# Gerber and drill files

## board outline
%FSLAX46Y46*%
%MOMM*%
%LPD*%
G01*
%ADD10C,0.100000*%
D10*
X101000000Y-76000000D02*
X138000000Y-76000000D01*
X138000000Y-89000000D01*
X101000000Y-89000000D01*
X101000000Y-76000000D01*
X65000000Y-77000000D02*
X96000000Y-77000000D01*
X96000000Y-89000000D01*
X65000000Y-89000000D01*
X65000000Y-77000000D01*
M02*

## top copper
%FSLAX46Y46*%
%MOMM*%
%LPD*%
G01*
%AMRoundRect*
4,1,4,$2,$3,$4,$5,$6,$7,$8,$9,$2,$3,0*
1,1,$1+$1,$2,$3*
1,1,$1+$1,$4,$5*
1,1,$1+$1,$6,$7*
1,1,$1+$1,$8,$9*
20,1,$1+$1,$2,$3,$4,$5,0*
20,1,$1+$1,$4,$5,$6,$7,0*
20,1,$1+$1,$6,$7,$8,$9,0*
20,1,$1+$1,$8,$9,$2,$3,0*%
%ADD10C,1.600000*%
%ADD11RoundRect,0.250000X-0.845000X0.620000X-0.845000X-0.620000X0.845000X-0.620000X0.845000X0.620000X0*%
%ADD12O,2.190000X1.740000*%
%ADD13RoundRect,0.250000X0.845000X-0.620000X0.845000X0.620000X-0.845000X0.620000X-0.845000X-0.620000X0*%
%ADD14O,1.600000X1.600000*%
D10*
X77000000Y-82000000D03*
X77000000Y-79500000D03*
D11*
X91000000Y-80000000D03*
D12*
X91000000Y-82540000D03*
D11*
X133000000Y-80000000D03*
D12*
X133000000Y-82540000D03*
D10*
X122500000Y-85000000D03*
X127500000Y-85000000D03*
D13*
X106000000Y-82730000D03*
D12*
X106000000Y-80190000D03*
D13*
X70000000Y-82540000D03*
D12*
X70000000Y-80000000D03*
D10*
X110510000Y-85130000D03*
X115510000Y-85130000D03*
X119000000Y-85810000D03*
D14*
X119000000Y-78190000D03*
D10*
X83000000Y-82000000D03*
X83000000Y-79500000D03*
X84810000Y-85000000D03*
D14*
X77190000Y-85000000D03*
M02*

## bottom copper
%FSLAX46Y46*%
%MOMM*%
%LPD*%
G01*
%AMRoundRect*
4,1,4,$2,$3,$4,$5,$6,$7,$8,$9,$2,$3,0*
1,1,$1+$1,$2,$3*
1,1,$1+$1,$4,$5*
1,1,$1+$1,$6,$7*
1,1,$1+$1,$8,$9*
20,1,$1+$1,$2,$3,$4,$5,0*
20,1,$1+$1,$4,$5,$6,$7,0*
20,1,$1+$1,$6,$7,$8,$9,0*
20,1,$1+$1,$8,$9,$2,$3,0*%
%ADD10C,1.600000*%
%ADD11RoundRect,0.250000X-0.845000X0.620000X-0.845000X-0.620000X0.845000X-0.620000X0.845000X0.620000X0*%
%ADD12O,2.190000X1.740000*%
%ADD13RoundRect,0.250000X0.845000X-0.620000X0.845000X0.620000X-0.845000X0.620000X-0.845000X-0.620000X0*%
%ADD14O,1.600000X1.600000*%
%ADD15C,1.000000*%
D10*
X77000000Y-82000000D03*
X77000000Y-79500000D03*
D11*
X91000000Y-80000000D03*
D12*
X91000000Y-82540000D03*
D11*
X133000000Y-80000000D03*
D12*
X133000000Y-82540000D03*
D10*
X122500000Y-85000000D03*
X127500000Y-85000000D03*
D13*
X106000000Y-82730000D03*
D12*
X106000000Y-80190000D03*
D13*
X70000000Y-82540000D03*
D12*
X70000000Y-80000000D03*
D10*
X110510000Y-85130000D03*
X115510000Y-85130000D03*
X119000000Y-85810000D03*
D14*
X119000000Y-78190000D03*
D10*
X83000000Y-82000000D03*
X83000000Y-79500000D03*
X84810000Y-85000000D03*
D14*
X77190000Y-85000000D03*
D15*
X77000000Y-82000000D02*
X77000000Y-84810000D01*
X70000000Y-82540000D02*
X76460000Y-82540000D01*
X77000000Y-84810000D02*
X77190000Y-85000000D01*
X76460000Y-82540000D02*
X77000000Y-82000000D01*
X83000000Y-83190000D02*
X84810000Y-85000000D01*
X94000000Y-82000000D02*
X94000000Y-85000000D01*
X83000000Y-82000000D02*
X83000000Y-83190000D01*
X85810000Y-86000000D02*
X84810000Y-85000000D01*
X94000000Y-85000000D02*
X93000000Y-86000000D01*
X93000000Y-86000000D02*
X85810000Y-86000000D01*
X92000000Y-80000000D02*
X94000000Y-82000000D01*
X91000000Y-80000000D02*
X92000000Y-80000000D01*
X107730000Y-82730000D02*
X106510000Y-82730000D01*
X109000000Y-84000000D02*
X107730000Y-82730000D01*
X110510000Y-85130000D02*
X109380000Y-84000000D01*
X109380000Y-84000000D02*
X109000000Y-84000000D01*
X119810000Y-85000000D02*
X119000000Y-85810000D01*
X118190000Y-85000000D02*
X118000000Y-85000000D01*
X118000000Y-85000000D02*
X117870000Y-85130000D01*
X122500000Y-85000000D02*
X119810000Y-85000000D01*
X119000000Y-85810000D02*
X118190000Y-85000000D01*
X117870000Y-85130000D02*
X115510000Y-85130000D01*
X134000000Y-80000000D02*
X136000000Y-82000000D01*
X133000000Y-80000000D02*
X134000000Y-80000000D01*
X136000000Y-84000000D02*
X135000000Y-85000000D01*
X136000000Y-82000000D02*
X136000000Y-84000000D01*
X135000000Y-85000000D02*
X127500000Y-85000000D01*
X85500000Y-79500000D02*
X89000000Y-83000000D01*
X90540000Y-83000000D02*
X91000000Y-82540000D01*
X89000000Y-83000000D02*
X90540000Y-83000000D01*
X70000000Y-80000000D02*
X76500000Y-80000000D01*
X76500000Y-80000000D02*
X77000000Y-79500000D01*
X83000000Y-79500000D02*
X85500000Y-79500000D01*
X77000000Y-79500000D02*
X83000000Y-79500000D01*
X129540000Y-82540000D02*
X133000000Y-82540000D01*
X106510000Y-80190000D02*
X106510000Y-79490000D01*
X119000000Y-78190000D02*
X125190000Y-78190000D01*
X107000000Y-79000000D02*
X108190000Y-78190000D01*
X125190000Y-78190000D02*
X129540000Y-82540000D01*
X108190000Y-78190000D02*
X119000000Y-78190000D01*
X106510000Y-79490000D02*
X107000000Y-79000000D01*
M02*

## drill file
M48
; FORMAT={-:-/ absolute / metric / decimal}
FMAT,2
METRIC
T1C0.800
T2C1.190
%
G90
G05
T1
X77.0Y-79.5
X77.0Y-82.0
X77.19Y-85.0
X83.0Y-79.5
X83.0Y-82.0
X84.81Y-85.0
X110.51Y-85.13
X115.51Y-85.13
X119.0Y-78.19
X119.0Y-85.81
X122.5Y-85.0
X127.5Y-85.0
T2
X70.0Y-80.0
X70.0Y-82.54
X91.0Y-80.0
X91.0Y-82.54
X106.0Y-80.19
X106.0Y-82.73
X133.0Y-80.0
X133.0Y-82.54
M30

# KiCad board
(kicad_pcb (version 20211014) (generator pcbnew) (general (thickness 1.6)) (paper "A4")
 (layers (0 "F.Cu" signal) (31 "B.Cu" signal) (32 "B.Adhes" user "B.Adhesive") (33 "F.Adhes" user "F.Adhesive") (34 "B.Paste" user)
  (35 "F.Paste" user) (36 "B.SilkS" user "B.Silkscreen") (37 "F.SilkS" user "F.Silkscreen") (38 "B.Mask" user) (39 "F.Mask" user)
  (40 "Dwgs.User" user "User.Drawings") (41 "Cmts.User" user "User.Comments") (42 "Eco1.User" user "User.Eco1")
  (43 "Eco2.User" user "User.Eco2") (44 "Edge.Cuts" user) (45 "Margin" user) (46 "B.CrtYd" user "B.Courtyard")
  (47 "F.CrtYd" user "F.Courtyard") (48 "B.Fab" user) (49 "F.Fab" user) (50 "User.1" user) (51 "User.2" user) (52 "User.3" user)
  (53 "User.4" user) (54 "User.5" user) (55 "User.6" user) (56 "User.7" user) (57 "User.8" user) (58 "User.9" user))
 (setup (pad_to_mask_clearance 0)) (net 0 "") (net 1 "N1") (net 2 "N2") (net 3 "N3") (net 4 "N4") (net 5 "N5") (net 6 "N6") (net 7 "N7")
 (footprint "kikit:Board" (layer "F.Cu") (at 67 77)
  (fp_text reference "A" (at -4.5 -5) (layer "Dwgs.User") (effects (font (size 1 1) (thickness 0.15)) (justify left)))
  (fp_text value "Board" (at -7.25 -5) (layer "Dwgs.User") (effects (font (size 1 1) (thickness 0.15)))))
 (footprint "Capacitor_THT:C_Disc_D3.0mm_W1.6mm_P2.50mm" (layer "F.Cu") (at 77 82 90)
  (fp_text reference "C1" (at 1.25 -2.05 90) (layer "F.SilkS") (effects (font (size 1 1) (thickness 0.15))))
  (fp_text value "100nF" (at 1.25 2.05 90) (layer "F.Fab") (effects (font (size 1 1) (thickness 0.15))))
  (pad "1" thru_hole circle (at 0 0 90) (size 1.6 1.6) (drill 0.8) (layers *.Cu *.Mask) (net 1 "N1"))
  (pad "2" thru_hole circle (at 2.5 0 90) (size 1.6 1.6) (drill 0.8) (layers *.Cu *.Mask) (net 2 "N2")))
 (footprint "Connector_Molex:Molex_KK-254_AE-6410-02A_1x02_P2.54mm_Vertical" (layer "F.Cu") (at 91 80 -90)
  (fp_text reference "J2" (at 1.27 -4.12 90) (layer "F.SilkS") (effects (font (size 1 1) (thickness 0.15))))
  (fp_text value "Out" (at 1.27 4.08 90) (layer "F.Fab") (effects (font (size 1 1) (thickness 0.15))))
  (pad "1" thru_hole roundrect (at 0 0 270) (size 1.74 2.19) (drill 1.19) (layers *.Cu *.Mask) (roundrect_rratio 0.143678) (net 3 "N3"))
  (pad "2" thru_hole oval (at 2.54 0 270) (size 1.74 2.19) (drill 1.19) (layers *.Cu *.Mask) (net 2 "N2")))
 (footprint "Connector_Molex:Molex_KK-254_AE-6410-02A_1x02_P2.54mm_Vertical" (layer "F.Cu") (at 133 80 -90)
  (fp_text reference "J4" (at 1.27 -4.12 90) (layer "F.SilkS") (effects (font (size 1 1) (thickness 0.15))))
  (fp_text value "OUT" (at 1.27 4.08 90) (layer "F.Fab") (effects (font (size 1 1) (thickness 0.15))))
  (pad "1" thru_hole roundrect (at 0 0 270) (size 1.74 2.19) (drill 1.19) (layers *.Cu *.Mask) (roundrect_rratio 0.143678) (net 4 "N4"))
  (pad "2" thru_hole oval (at 2.54 0 270) (size 1.74 2.19) (drill 1.19) (layers *.Cu *.Mask) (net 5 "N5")))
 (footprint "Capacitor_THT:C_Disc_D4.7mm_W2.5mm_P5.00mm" (layer "F.Cu") (at 122.5 85)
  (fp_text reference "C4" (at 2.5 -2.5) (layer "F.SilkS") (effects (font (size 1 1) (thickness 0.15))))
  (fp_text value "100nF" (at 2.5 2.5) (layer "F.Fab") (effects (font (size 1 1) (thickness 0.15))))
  (pad "1" thru_hole circle (at 0 0) (size 1.6 1.6) (drill 0.8) (layers *.Cu *.Mask) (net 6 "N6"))
  (pad "2" thru_hole circle (at 5 0) (size 1.6 1.6) (drill 0.8) (layers *.Cu *.Mask) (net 4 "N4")))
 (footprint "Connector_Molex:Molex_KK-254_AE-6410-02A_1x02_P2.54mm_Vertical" (layer "F.Cu") (at 106 82.73 90)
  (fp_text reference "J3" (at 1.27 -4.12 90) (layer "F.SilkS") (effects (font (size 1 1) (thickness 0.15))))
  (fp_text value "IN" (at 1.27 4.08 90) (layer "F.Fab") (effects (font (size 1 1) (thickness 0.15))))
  (pad "1" thru_hole roundrect (at 0 0 90) (size 1.74 2.19) (drill 1.19) (layers *.Cu *.Mask) (roundrect_rratio 0.143678) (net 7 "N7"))
  (pad "2" thru_hole oval (at 2.54 0 90) (size 1.74 2.19) (drill 1.19) (layers *.Cu *.Mask) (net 5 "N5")))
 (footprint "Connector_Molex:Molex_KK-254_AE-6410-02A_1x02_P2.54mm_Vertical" (layer "F.Cu") (at 70 82.54 90)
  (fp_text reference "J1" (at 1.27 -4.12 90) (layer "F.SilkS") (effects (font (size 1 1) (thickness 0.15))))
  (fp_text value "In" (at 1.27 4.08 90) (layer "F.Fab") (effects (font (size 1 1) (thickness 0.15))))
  (pad "1" thru_hole roundrect (at 0 0 90) (size 1.74 2.19) (drill 1.19) (layers *.Cu *.Mask) (roundrect_rratio 0.143678) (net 1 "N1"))
  (pad "2" thru_hole oval (at 2.54 0 90) (size 1.74 2.19) (drill 1.19) (layers *.Cu *.Mask) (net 2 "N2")))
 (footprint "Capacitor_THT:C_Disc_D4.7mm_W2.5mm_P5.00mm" (layer "F.Cu") (at 110.51 85.13)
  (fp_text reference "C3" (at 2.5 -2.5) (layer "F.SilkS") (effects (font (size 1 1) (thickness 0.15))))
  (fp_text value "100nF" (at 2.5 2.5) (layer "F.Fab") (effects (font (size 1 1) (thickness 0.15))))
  (pad "1" thru_hole circle (at 0 0) (size 1.6 1.6) (drill 0.8) (layers *.Cu *.Mask) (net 7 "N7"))
  (pad "2" thru_hole circle (at 5 0) (size 1.6 1.6) (drill 0.8) (layers *.Cu *.Mask) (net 6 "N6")))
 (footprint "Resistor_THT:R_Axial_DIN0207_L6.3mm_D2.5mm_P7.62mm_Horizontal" (layer "F.Cu") (at 119 85.81 90)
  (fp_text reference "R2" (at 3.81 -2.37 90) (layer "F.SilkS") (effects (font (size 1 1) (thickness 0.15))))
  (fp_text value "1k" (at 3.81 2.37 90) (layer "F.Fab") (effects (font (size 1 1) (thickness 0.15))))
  (pad "1" thru_hole circle (at 0 0 90) (size 1.6 1.6) (drill 0.8) (layers *.Cu *.Mask) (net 6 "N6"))
  (pad "2" thru_hole oval (at 7.62 0 90) (size 1.6 1.6) (drill 0.8) (layers *.Cu *.Mask) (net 5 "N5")))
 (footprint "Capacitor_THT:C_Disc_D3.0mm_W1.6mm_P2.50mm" (layer "F.Cu") (at 83 82 90)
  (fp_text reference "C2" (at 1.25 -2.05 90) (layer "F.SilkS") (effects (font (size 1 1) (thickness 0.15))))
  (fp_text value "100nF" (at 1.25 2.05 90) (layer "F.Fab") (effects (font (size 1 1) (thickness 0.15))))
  (pad "1" thru_hole circle (at 0 0 90) (size 1.6 1.6) (drill 0.8) (layers *.Cu *.Mask) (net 3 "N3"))
  (pad "2" thru_hole circle (at 2.5 0 90) (size 1.6 1.6) (drill 0.8) (layers *.Cu *.Mask) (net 2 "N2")))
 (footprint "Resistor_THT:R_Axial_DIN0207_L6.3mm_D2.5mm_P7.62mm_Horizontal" (layer "F.Cu") (at 84.81 85 180)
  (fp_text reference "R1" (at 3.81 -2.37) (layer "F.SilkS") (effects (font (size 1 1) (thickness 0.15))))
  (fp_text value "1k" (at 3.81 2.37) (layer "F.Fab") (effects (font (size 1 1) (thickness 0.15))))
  (pad "1" thru_hole circle (at 0 0 180) (size 1.6 1.6) (drill 0.8) (layers *.Cu *.Mask) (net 3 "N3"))
  (pad "2" thru_hole oval (at 7.62 0 180) (size 1.6 1.6) (drill 0.8) (layers *.Cu *.Mask) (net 1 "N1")))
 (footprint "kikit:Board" (layer "F.Cu") (at 105 76)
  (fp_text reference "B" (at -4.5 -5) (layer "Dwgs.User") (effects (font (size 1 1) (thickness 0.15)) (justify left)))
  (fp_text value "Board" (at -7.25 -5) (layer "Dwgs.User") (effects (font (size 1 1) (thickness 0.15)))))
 (gr_rect (start 101 76) (end 138 89) (layer "Edge.Cuts") (width 0.1) (fill none))
 (gr_rect (start 96 89) (end 65 77) (layer "Edge.Cuts") (width 0.1) (fill none))
 (segment (start 77 82) (end 77 84.81) (width 1) (layer "B.Cu") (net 1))
 (segment (start 70 82.54) (end 76.46 82.54) (width 1) (layer "B.Cu") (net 1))
 (segment (start 77 84.81) (end 77.19 85) (width 1) (layer "B.Cu") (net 1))
 (segment (start 76.46 82.54) (end 77 82) (width 1) (layer "B.Cu") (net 1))
 (segment (start 83 83.19) (end 84.81 85) (width 1) (layer "B.Cu") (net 3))
 (segment (start 94 82) (end 94 85) (width 1) (layer "B.Cu") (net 3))
 (segment (start 83 82) (end 83 83.19) (width 1) (layer "B.Cu") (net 3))
 (segment (start 85.81 86) (end 84.81 85) (width 1) (layer "B.Cu") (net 3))
 (segment (start 94 85) (end 93 86) (width 1) (layer "B.Cu") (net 3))
 (segment (start 93 86) (end 85.81 86) (width 1) (layer "B.Cu") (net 3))
 (segment (start 92 80) (end 94 82) (width 1) (layer "B.Cu") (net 3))
 (segment (start 91 80) (end 92 80) (width 1) (layer "B.Cu") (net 3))
 (segment (start 107.73 82.73) (end 106.51 82.73) (width 1) (layer "B.Cu") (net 7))
 (segment (start 109 84) (end 107.73 82.73) (width 1) (layer "B.Cu") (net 7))
 (segment (start 110.51 85.13) (end 109.38 84) (width 1) (layer "B.Cu") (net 7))
 (segment (start 109.38 84) (end 109 84) (width 1) (layer "B.Cu") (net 7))
 (segment (start 119.81 85) (end 119 85.81) (width 1) (layer "B.Cu") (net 6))
 (segment (start 118.19 85) (end 118 85) (width 1) (layer "B.Cu") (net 6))
 (segment (start 118 85) (end 117.87 85.13) (width 1) (layer "B.Cu") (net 6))
 (segment (start 122.5 85) (end 119.81 85) (width 1) (layer "B.Cu") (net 6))
 (segment (start 119 85.81) (end 118.19 85) (width 1) (layer "B.Cu") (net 6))
 (segment (start 117.87 85.13) (end 115.51 85.13) (width 1) (layer "B.Cu") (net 6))
 (segment (start 134 80) (end 136 82) (width 1) (layer "B.Cu") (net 4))
 (segment (start 133 80) (end 134 80) (width 1) (layer "B.Cu") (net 4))
 (segment (start 136 84) (end 135 85) (width 1) (layer "B.Cu") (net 4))
 (segment (start 136 82) (end 136 84) (width 1) (layer "B.Cu") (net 4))
 (segment (start 135 85) (end 127.5 85) (width 1) (layer "B.Cu") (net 4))
 (segment (start 85.5 79.5) (end 89 83) (width 1) (layer "B.Cu") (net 2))
 (segment (start 90.54 83) (end 91 82.54) (width 1) (layer "B.Cu") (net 2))
 (segment (start 89 83) (end 90.54 83) (width 1) (layer "B.Cu") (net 2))
 (segment (start 70 80) (end 76.5 80) (width 1) (layer "B.Cu") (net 2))
 (segment (start 76.5 80) (end 77 79.5) (width 1) (layer "B.Cu") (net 2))
 (segment (start 83 79.5) (end 85.5 79.5) (width 1) (layer "B.Cu") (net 2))
 (segment (start 77 79.5) (end 83 79.5) (width 1) (layer "B.Cu") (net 2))
 (segment (start 129.54 82.54) (end 133 82.54) (width 1) (layer "B.Cu") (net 5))
 (segment (start 106.51 80.19) (end 106.51 79.49) (width 1) (layer "B.Cu") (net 5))
 (segment (start 119 78.19) (end 125.19 78.19) (width 1) (layer "B.Cu") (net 5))
 (segment (start 107 79) (end 108.19 78.19) (width 1) (layer "B.Cu") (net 5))
 (segment (start 125.19 78.19) (end 129.54 82.54) (width 1) (layer "B.Cu") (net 5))
 (segment (start 108.19 78.19) (end 119 78.19) (width 1) (layer "B.Cu") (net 5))
 (segment (start 106.51 79.49) (end 107 79) (width 1) (layer "B.Cu") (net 5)))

